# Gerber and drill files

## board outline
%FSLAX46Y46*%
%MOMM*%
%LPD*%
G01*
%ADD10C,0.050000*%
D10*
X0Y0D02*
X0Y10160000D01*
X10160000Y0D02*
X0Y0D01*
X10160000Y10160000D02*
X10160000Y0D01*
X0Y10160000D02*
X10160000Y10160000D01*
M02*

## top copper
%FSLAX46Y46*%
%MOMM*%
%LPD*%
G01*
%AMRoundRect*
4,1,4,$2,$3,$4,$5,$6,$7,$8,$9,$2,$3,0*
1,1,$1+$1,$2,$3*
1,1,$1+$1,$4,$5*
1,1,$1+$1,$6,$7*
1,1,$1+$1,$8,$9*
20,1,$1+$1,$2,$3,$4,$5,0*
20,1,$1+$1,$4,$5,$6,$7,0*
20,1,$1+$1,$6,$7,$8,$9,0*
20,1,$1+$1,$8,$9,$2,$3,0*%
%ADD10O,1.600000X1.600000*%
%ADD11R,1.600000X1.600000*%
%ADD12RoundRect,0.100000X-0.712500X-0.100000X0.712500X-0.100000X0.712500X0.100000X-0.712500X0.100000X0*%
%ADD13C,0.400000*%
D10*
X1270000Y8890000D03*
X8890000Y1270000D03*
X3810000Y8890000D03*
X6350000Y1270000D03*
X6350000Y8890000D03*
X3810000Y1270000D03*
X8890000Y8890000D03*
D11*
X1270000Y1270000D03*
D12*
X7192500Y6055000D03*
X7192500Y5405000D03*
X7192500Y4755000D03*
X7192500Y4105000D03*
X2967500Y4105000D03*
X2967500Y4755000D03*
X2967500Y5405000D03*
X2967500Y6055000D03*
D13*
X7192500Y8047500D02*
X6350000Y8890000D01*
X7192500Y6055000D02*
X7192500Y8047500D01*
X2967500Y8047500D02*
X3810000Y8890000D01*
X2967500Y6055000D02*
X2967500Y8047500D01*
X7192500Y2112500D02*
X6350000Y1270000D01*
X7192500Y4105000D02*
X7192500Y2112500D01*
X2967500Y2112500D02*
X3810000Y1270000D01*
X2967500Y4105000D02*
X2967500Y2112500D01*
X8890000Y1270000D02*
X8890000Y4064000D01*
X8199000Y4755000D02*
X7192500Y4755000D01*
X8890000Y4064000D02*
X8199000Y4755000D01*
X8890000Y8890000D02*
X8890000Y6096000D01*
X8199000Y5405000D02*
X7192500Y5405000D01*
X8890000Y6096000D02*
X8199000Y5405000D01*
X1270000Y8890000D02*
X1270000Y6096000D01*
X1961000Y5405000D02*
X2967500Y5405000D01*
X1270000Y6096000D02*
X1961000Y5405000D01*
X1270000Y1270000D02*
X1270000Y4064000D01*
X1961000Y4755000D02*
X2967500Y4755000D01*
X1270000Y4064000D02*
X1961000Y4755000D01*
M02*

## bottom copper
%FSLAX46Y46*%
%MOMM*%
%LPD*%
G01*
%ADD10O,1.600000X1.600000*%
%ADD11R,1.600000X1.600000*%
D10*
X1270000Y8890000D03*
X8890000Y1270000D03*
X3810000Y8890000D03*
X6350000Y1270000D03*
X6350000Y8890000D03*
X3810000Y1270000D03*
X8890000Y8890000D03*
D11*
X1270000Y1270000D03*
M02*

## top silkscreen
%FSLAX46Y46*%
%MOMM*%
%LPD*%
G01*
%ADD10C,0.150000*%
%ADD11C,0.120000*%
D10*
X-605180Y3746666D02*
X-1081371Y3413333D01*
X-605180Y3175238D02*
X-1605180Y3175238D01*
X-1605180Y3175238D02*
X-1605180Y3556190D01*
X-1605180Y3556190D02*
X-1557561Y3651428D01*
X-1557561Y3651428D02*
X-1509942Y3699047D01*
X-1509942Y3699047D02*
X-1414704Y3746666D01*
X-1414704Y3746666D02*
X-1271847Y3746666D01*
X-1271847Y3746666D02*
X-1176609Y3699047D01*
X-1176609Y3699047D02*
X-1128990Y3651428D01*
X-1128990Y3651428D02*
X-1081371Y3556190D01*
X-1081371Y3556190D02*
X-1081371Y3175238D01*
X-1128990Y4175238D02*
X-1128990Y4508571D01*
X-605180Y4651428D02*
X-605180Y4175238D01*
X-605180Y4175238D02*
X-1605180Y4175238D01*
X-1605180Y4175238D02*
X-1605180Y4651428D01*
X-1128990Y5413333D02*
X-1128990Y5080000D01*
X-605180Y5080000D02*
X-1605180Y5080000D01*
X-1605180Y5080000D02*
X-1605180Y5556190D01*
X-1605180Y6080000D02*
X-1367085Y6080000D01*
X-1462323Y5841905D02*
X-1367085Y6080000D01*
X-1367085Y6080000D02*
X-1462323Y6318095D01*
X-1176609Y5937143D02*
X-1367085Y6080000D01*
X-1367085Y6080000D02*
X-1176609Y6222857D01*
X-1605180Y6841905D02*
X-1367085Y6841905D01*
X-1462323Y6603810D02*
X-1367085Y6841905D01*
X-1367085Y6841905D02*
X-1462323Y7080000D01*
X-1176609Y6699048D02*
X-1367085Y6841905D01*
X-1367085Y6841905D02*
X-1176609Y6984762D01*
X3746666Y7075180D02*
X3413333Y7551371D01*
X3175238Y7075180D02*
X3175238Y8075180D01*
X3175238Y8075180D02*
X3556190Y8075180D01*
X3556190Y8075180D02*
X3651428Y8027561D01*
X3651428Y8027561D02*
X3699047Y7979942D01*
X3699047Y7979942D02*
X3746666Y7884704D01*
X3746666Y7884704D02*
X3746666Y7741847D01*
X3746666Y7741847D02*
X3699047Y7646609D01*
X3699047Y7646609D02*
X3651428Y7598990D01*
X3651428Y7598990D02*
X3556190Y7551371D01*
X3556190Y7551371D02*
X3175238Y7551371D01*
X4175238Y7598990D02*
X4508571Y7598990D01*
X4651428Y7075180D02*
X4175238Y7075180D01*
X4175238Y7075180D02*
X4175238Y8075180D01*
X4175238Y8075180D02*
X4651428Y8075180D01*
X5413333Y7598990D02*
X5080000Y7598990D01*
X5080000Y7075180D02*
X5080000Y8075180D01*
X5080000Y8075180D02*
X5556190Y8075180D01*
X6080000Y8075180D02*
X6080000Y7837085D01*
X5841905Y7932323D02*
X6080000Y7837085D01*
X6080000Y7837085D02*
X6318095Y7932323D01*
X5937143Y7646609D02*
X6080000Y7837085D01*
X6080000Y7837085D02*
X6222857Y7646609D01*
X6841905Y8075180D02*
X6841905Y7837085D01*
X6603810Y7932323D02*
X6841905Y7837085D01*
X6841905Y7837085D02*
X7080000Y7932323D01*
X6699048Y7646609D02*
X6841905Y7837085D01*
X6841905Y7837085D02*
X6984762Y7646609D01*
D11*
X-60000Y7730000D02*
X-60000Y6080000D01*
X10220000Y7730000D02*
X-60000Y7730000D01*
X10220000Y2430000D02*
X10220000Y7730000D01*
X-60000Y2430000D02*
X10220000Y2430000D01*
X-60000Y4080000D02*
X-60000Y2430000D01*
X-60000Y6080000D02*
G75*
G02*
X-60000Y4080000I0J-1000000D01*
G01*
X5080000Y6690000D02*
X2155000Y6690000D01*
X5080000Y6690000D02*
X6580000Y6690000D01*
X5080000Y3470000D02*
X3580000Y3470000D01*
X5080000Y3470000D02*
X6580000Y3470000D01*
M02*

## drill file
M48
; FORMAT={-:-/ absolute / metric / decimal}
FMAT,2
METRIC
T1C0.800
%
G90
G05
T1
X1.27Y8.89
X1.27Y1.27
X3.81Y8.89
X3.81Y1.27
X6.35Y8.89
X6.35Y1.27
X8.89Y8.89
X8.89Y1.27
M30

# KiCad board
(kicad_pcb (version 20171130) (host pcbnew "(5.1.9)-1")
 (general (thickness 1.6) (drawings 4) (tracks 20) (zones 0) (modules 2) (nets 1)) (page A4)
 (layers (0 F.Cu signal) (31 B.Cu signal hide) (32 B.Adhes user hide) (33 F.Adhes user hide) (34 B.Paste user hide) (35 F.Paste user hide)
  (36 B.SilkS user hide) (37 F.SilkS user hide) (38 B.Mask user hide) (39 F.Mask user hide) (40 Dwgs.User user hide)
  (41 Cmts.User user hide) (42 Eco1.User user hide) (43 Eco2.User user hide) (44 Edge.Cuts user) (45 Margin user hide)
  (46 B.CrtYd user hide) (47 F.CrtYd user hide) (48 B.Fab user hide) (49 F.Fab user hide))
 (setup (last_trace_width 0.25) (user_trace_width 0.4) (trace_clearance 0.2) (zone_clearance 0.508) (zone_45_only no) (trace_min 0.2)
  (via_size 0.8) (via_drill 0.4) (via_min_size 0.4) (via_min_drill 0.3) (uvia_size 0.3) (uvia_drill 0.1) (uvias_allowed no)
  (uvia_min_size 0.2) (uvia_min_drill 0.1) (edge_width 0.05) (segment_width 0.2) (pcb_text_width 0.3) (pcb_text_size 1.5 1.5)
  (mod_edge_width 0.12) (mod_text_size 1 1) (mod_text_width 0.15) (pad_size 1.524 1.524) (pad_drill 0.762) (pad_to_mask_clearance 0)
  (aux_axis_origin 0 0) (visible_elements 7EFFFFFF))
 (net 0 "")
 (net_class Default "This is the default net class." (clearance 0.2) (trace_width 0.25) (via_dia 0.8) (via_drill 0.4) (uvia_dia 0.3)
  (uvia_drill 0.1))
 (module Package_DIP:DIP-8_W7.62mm (layer F.Cu) (at 1.27 -1.27 90)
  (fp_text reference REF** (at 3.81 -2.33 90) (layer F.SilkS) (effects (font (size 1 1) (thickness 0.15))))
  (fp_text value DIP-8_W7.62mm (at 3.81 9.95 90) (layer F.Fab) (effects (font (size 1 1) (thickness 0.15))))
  (fp_line (start 6.46 -1.33) (end 4.81 -1.33) (layer F.SilkS) (width 0.12))
  (fp_line (start 6.46 8.95) (end 6.46 -1.33) (layer F.SilkS) (width 0.12))
  (fp_line (start 1.16 8.95) (end 6.46 8.95) (layer F.SilkS) (width 0.12))
  (fp_line (start 1.16 -1.33) (end 1.16 8.95) (layer F.SilkS) (width 0.12))
  (fp_line (start 2.81 -1.33) (end 1.16 -1.33) (layer F.SilkS) (width 0.12))
  (fp_arc (start 3.81 -1.33) (end 2.81 -1.33) (angle -180) (layer F.SilkS) (width 0.12))
  (pad 8 thru_hole oval (at 7.62 0 90) (size 1.6 1.6) (drill 0.8) (layers *.Cu *.Mask))
  (pad 4 thru_hole oval (at 0 7.62 90) (size 1.6 1.6) (drill 0.8) (layers *.Cu *.Mask))
  (pad 7 thru_hole oval (at 7.62 2.54 90) (size 1.6 1.6) (drill 0.8) (layers *.Cu *.Mask))
  (pad 3 thru_hole oval (at 0 5.08 90) (size 1.6 1.6) (drill 0.8) (layers *.Cu *.Mask))
  (pad 6 thru_hole oval (at 7.62 5.08 90) (size 1.6 1.6) (drill 0.8) (layers *.Cu *.Mask))
  (pad 2 thru_hole oval (at 0 2.54 90) (size 1.6 1.6) (drill 0.8) (layers *.Cu *.Mask))
  (pad 5 thru_hole oval (at 7.62 7.62 90) (size 1.6 1.6) (drill 0.8) (layers *.Cu *.Mask))
  (pad 1 thru_hole rect (at 0 0 90) (size 1.6 1.6) (drill 0.8) (layers *.Cu *.Mask)))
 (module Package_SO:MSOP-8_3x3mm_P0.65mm (layer F.Cu) (at 5.08 -5.08)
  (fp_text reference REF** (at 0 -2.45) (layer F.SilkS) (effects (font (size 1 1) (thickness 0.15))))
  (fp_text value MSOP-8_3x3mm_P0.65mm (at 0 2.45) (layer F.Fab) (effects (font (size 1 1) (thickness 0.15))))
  (fp_line (start 0 -1.61) (end -2.925 -1.61) (layer F.SilkS) (width 0.12))
  (fp_line (start 0 -1.61) (end 1.5 -1.61) (layer F.SilkS) (width 0.12))
  (fp_line (start 0 1.61) (end -1.5 1.61) (layer F.SilkS) (width 0.12))
  (fp_line (start 0 1.61) (end 1.5 1.61) (layer F.SilkS) (width 0.12))
  (pad 8 smd roundrect (at 2.1125 -0.975) (size 1.625 0.4) (layers F.Cu F.Paste F.Mask) (roundrect_rratio 0.25))
  (pad 7 smd roundrect (at 2.1125 -0.325) (size 1.625 0.4) (layers F.Cu F.Paste F.Mask) (roundrect_rratio 0.25))
  (pad 6 smd roundrect (at 2.1125 0.325) (size 1.625 0.4) (layers F.Cu F.Paste F.Mask) (roundrect_rratio 0.25))
  (pad 5 smd roundrect (at 2.1125 0.975) (size 1.625 0.4) (layers F.Cu F.Paste F.Mask) (roundrect_rratio 0.25))
  (pad 4 smd roundrect (at -2.1125 0.975) (size 1.625 0.4) (layers F.Cu F.Paste F.Mask) (roundrect_rratio 0.25))
  (pad 3 smd roundrect (at -2.1125 0.325) (size 1.625 0.4) (layers F.Cu F.Paste F.Mask) (roundrect_rratio 0.25))
  (pad 2 smd roundrect (at -2.1125 -0.325) (size 1.625 0.4) (layers F.Cu F.Paste F.Mask) (roundrect_rratio 0.25))
  (pad 1 smd roundrect (at -2.1125 -0.975) (size 1.625 0.4) (layers F.Cu F.Paste F.Mask) (roundrect_rratio 0.25)))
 (gr_line (start 0 0) (end 0 -10.16) (layer Edge.Cuts) (width 0.05))
 (gr_line (start 10.16 0) (end 0 0) (layer Edge.Cuts) (width 0.05))
 (gr_line (start 10.16 -10.16) (end 10.16 0) (layer Edge.Cuts) (width 0.05))
 (gr_line (start 0 -10.16) (end 10.16 -10.16) (layer Edge.Cuts) (width 0.05))
 (segment (start 7.1925 -8.0475) (end 6.35 -8.89) (width 0.4) (layer F.Cu) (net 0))
 (segment (start 7.1925 -6.055) (end 7.1925 -8.0475) (width 0.4) (layer F.Cu) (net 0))
 (segment (start 2.9675 -8.0475) (end 3.81 -8.89) (width 0.4) (layer F.Cu) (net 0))
 (segment (start 2.9675 -6.055) (end 2.9675 -8.0475) (width 0.4) (layer F.Cu) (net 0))
 (segment (start 7.1925 -2.1125) (end 6.35 -1.27) (width 0.4) (layer F.Cu) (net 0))
 (segment (start 7.1925 -4.105) (end 7.1925 -2.1125) (width 0.4) (layer F.Cu) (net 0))
 (segment (start 2.9675 -2.1125) (end 3.81 -1.27) (width 0.4) (layer F.Cu) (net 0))
 (segment (start 2.9675 -4.105) (end 2.9675 -2.1125) (width 0.4) (layer F.Cu) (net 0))
 (segment (start 8.89 -1.27) (end 8.89 -4.064) (width 0.4) (layer F.Cu) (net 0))
 (segment (start 8.199 -4.755) (end 7.1925 -4.755) (width 0.4) (layer F.Cu) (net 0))
 (segment (start 8.89 -4.064) (end 8.199 -4.755) (width 0.4) (layer F.Cu) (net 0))
 (segment (start 8.89 -8.89) (end 8.89 -6.096) (width 0.4) (layer F.Cu) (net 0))
 (segment (start 8.199 -5.405) (end 7.1925 -5.405) (width 0.4) (layer F.Cu) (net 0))
 (segment (start 8.89 -6.096) (end 8.199 -5.405) (width 0.4) (layer F.Cu) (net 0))
 (segment (start 1.27 -8.89) (end 1.27 -6.096) (width 0.4) (layer F.Cu) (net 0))
 (segment (start 1.961 -5.405) (end 2.9675 -5.405) (width 0.4) (layer F.Cu) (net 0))
 (segment (start 1.27 -6.096) (end 1.961 -5.405) (width 0.4) (layer F.Cu) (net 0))
 (segment (start 1.27 -1.27) (end 1.27 -4.064) (width 0.4) (layer F.Cu) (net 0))
 (segment (start 1.961 -4.755) (end 2.9675 -4.755) (width 0.4) (layer F.Cu) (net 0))
 (segment (start 1.27 -4.064) (end 1.961 -4.755) (width 0.4) (layer F.Cu) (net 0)))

